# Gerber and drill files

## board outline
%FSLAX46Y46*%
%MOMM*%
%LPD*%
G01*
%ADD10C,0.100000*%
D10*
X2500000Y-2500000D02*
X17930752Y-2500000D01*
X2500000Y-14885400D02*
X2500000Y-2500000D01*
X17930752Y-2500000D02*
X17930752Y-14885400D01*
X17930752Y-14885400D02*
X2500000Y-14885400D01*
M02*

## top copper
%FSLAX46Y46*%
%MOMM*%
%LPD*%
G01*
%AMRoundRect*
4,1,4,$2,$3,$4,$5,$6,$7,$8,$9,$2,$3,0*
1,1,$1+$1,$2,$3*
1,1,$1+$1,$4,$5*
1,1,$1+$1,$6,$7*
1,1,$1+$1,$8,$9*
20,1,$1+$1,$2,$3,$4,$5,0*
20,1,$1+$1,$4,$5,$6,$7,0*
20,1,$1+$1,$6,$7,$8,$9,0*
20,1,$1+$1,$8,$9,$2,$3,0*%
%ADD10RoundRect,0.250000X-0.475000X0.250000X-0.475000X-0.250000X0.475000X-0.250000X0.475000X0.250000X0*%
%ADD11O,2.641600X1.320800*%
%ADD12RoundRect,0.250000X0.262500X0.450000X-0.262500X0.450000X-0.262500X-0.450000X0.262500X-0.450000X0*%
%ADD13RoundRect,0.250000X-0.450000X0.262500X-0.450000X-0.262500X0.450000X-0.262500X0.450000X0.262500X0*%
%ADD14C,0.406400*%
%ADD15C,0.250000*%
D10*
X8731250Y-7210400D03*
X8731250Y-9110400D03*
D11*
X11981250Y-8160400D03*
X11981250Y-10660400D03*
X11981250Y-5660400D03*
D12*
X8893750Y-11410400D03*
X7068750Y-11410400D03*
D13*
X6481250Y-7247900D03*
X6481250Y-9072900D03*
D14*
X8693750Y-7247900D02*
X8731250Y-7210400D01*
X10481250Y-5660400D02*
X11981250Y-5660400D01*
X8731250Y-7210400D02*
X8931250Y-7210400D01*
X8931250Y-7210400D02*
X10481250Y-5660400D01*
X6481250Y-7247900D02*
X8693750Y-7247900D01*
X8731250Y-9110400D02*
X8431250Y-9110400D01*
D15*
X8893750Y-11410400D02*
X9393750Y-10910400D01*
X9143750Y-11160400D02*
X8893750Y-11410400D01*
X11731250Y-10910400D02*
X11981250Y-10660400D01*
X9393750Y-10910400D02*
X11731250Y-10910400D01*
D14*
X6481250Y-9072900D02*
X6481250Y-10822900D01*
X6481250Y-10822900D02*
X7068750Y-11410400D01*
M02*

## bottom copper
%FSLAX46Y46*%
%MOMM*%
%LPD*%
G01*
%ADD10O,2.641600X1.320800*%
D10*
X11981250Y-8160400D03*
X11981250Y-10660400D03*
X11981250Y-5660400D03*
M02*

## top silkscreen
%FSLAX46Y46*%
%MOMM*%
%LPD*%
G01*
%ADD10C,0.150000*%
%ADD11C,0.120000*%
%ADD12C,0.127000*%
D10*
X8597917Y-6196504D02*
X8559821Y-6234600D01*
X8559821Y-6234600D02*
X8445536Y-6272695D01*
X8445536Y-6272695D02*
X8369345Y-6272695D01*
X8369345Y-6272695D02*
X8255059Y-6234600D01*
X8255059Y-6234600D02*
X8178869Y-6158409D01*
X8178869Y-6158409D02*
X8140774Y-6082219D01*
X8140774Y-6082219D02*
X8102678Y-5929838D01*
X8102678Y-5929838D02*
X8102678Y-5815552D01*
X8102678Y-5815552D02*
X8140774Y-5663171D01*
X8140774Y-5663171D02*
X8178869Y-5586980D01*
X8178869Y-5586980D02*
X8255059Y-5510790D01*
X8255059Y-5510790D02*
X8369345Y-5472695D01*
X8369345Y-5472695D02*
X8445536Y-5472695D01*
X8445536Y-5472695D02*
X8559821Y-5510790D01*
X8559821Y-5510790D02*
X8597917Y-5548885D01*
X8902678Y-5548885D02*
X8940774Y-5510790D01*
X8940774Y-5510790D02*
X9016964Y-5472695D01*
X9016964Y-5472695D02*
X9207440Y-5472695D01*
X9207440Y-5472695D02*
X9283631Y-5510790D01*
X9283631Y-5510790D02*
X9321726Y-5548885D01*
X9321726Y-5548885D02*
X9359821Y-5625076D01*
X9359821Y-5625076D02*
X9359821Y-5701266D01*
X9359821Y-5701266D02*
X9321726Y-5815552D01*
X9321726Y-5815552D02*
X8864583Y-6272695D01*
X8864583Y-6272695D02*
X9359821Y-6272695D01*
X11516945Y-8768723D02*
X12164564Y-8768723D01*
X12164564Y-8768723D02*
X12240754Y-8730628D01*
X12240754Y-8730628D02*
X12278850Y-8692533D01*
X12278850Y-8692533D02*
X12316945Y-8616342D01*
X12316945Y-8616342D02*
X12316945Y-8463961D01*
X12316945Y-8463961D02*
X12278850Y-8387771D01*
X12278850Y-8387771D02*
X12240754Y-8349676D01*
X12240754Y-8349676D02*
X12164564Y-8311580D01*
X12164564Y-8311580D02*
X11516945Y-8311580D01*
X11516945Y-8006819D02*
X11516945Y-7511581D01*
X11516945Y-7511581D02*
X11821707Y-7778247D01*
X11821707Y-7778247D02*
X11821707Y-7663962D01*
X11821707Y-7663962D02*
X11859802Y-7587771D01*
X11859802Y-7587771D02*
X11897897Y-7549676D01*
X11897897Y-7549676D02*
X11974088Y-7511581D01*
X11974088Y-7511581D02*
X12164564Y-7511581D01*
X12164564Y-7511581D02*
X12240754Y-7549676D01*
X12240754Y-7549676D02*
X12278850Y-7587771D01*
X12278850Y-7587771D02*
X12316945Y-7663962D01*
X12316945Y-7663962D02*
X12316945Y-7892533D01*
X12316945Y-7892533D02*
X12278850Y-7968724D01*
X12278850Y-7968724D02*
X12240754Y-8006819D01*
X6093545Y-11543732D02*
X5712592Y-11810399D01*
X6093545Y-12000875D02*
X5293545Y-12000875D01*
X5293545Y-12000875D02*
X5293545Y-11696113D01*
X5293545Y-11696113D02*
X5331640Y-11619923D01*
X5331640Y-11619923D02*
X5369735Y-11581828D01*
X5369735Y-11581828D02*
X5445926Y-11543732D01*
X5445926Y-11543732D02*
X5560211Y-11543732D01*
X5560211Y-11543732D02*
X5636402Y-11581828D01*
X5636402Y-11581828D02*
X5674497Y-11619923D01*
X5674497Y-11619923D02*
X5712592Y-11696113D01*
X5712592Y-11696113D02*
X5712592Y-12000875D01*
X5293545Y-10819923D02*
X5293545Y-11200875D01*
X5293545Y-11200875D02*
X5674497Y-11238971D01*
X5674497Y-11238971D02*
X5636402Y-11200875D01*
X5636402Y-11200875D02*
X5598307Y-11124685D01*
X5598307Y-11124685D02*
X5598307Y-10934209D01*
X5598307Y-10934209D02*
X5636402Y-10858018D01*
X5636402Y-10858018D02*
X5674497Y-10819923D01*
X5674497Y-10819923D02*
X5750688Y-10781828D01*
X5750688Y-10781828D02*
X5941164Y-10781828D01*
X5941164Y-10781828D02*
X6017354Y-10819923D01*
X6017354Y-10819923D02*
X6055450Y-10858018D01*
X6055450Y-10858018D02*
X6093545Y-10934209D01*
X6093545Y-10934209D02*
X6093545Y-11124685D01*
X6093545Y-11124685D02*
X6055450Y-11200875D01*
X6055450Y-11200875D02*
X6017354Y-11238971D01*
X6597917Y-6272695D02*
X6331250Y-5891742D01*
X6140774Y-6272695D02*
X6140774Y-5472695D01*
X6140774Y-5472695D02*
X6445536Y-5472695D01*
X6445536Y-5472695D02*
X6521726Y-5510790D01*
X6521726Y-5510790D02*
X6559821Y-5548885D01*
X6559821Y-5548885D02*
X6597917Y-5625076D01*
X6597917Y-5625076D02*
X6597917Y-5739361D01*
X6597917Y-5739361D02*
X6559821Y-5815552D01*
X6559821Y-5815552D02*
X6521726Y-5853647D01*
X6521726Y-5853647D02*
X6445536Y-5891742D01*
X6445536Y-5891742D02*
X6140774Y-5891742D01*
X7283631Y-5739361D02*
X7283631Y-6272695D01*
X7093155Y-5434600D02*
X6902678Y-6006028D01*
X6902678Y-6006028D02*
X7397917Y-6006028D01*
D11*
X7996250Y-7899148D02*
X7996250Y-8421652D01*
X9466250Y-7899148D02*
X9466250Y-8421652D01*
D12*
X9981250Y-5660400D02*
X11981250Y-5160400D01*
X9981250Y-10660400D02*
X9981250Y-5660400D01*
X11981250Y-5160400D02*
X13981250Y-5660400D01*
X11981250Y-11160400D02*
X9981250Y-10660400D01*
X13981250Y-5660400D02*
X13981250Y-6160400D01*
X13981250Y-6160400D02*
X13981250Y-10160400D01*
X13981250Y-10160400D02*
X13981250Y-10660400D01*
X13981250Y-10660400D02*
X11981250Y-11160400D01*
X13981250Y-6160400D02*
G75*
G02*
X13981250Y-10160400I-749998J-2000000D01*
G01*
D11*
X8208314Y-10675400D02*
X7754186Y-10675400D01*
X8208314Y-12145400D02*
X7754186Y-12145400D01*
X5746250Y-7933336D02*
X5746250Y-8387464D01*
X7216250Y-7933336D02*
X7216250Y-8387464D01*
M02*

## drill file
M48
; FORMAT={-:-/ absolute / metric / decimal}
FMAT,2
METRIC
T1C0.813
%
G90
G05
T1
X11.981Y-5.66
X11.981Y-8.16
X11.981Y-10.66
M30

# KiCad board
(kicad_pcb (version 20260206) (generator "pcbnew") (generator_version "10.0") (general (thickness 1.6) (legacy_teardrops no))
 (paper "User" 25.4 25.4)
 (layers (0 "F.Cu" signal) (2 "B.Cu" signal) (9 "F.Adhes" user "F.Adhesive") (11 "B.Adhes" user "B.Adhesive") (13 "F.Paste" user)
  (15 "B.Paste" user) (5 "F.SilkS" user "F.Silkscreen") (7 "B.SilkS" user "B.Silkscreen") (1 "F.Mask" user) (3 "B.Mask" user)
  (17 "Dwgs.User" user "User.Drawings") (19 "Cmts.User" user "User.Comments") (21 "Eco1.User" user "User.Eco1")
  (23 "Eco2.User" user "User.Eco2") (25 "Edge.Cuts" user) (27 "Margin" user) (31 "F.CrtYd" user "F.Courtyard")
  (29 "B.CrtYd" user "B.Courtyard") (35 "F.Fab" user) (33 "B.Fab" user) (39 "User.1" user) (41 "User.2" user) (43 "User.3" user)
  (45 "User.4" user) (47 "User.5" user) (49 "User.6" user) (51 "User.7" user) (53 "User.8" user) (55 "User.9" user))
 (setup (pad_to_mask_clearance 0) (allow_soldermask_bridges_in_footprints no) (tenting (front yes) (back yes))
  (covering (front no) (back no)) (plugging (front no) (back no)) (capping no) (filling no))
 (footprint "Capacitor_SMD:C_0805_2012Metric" (layer "F.Cu") (at 8.73125 8.1604 -90)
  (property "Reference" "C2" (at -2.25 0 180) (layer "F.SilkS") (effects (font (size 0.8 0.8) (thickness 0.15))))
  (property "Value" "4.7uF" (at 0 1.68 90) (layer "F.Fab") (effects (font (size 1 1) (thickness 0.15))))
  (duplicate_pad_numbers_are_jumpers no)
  (fp_line (start -0.261252 0.735) (end 0.261252 0.735) (stroke (width 0.12) (type solid)) (layer "F.SilkS"))
  (fp_line (start -0.261252 -0.735) (end 0.261252 -0.735) (stroke (width 0.12) (type solid)) (layer "F.SilkS"))
  (pad "1" smd roundrect (at -0.95 0 270) (size 1 1.45) (layers "F.Cu" "F.Mask" "F.Paste") (roundrect_rratio 0.25) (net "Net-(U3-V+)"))
  (pad "2" smd roundrect (at 0.95 0 270) (size 1 1.45) (layers "F.Cu" "F.Mask" "F.Paste") (roundrect_rratio 0.25) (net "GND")))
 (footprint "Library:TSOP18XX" (layer "F.Cu") (at 11.95465 8.1592 90)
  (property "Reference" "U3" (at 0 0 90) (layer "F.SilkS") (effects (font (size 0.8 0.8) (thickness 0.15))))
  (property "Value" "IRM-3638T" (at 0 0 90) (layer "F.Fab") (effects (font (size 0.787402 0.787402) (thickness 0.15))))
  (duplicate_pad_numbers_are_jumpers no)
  (fp_line (start 2.4988 -1.9734) (end 2.9988 0.0266) (stroke (width 0.127) (type solid)) (layer "F.SilkS"))
  (fp_line (start -2.5012 -1.9734) (end 2.4988 -1.9734) (stroke (width 0.127) (type solid)) (layer "F.SilkS"))
  (fp_line (start 2.9988 0.0266) (end 2.4988 2.0266) (stroke (width 0.127) (type solid)) (layer "F.SilkS"))
  (fp_line (start -3.0012 0.0266) (end -2.5012 -1.9734) (stroke (width 0.127) (type solid)) (layer "F.SilkS"))
  (fp_line (start 2.4988 2.0266) (end 1.9988 2.0266) (stroke (width 0.127) (type solid)) (layer "F.SilkS"))
  (fp_line (start 1.9988 2.0266) (end -2.0012 2.0266) (stroke (width 0.127) (type solid)) (layer "F.SilkS"))
  (fp_line (start -2.0012 2.0266) (end -2.5012 2.0266) (stroke (width 0.127) (type solid)) (layer "F.SilkS"))
  (fp_line (start -2.5012 2.0266) (end -3.0012 0.0266) (stroke (width 0.127) (type solid)) (layer "F.SilkS"))
  (fp_arc (start 1.9988 2.0266) (mid -0.0012 3.412602) (end -2.0012 2.0266) (stroke (width 0.127) (type solid)) (layer "F.SilkS"))
  (pad "GND" thru_hole oval (at -0.0012 0.0266 90) (size 1.3208 2.6416) (drill 0.8128) (layers "*.Cu" "*.Mask") (remove_unused_layers no)
   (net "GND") (solder_mask_margin 0.102))
  (pad "OUT" thru_hole oval (at -2.5012 0.0266 90) (size 1.3208 2.6416) (drill 0.8128) (layers "*.Cu" "*.Mask") (remove_unused_layers no)
   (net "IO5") (solder_mask_margin 0.102))
  (pad "VCC" thru_hole oval (at 2.4988 0.0266 90) (size 1.3208 2.6416) (drill 0.8128) (layers "*.Cu" "*.Mask") (remove_unused_layers no)
   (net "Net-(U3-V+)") (solder_mask_margin 0.102)))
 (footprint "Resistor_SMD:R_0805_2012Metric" (layer "F.Cu") (at 7.98125 11.4104 180)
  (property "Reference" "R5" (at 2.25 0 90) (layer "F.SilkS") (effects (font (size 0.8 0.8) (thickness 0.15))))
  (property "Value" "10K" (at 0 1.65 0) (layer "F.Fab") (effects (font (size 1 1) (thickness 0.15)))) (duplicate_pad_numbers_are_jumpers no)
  (fp_line (start -0.227064 0.735) (end 0.227064 0.735) (stroke (width 0.12) (type solid)) (layer "F.SilkS"))
  (fp_line (start -0.227064 -0.735) (end 0.227064 -0.735) (stroke (width 0.12) (type solid)) (layer "F.SilkS"))
  (pad "1" smd roundrect (at -0.9125 0 180) (size 1.025 1.4) (layers "F.Cu" "F.Mask" "F.Paste") (roundrect_rratio 0.243902439) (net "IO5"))
  (pad "2" smd roundrect (at 0.9125 0 180) (size 1.025 1.4) (layers "F.Cu" "F.Mask" "F.Paste") (roundrect_rratio 0.243902439) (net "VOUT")))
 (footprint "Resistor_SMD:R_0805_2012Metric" (layer "F.Cu") (at 6.48125 8.1604 -90)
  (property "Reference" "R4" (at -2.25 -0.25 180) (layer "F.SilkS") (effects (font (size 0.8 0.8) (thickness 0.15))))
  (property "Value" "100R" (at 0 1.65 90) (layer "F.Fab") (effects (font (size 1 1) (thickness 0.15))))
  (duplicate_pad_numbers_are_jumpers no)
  (fp_line (start -0.227064 0.735) (end 0.227064 0.735) (stroke (width 0.12) (type solid)) (layer "F.SilkS"))
  (fp_line (start -0.227064 -0.735) (end 0.227064 -0.735) (stroke (width 0.12) (type solid)) (layer "F.SilkS"))
  (pad "1" smd roundrect (at -0.9125 0 270) (size 1.025 1.4) (layers "F.Cu" "F.Mask" "F.Paste") (roundrect_rratio 0.243902439)
   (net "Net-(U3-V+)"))
  (pad "2" smd roundrect (at 0.9125 0 270) (size 1.025 1.4) (layers "F.Cu" "F.Mask" "F.Paste") (roundrect_rratio 0.243902439) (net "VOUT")))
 (gr_line (start 2.5 2.5) (end 17.930752 2.5) (stroke (width 0.1) (type default)) (layer "Edge.Cuts"))
 (gr_line (start 2.5 14.8854) (end 2.5 2.5) (stroke (width 0.1) (type default)) (layer "Edge.Cuts"))
 (gr_line (start 17.930752 2.5) (end 17.930752 14.8854) (stroke (width 0.1) (type default)) (layer "Edge.Cuts"))
 (gr_line (start 17.930752 14.8854) (end 2.5 14.8854) (stroke (width 0.1) (type default)) (layer "Edge.Cuts"))
 (segment (start 8.69375 7.2479) (end 8.73125 7.2104) (width 0.4064) (layer "F.Cu") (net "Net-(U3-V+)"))
 (segment (start 10.48125 5.6604) (end 11.98125 5.6604) (width 0.4064) (layer "F.Cu") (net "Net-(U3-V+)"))
 (segment (start 8.73125 7.2104) (end 8.93125 7.2104) (width 0.4064) (layer "F.Cu") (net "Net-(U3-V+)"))
 (segment (start 8.93125 7.2104) (end 10.48125 5.6604) (width 0.4064) (layer "F.Cu") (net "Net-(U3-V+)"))
 (segment (start 6.48125 7.2479) (end 8.69375 7.2479) (width 0.4064) (layer "F.Cu") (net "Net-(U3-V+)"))
 (segment (start 8.73125 9.1104) (end 8.43125 9.1104) (width 0.4064) (layer "F.Cu") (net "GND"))
 (segment (start 8.89375 11.4104) (end 9.39375 10.9104) (width 0.25) (layer "F.Cu") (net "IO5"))
 (segment (start 9.14375 11.1604) (end 8.89375 11.4104) (width 0.25) (layer "F.Cu") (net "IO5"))
 (segment (start 11.73125 10.9104) (end 11.98125 10.6604) (width 0.25) (layer "F.Cu") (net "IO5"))
 (segment (start 9.39375 10.9104) (end 11.73125 10.9104) (width 0.25) (layer "F.Cu") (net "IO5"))
 (segment (start 6.48125 9.0729) (end 6.48125 10.8229) (width 0.4064) (layer "F.Cu") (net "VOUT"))
 (segment (start 6.48125 10.8229) (end 7.06875 11.4104) (width 0.4064) (layer "F.Cu") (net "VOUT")))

